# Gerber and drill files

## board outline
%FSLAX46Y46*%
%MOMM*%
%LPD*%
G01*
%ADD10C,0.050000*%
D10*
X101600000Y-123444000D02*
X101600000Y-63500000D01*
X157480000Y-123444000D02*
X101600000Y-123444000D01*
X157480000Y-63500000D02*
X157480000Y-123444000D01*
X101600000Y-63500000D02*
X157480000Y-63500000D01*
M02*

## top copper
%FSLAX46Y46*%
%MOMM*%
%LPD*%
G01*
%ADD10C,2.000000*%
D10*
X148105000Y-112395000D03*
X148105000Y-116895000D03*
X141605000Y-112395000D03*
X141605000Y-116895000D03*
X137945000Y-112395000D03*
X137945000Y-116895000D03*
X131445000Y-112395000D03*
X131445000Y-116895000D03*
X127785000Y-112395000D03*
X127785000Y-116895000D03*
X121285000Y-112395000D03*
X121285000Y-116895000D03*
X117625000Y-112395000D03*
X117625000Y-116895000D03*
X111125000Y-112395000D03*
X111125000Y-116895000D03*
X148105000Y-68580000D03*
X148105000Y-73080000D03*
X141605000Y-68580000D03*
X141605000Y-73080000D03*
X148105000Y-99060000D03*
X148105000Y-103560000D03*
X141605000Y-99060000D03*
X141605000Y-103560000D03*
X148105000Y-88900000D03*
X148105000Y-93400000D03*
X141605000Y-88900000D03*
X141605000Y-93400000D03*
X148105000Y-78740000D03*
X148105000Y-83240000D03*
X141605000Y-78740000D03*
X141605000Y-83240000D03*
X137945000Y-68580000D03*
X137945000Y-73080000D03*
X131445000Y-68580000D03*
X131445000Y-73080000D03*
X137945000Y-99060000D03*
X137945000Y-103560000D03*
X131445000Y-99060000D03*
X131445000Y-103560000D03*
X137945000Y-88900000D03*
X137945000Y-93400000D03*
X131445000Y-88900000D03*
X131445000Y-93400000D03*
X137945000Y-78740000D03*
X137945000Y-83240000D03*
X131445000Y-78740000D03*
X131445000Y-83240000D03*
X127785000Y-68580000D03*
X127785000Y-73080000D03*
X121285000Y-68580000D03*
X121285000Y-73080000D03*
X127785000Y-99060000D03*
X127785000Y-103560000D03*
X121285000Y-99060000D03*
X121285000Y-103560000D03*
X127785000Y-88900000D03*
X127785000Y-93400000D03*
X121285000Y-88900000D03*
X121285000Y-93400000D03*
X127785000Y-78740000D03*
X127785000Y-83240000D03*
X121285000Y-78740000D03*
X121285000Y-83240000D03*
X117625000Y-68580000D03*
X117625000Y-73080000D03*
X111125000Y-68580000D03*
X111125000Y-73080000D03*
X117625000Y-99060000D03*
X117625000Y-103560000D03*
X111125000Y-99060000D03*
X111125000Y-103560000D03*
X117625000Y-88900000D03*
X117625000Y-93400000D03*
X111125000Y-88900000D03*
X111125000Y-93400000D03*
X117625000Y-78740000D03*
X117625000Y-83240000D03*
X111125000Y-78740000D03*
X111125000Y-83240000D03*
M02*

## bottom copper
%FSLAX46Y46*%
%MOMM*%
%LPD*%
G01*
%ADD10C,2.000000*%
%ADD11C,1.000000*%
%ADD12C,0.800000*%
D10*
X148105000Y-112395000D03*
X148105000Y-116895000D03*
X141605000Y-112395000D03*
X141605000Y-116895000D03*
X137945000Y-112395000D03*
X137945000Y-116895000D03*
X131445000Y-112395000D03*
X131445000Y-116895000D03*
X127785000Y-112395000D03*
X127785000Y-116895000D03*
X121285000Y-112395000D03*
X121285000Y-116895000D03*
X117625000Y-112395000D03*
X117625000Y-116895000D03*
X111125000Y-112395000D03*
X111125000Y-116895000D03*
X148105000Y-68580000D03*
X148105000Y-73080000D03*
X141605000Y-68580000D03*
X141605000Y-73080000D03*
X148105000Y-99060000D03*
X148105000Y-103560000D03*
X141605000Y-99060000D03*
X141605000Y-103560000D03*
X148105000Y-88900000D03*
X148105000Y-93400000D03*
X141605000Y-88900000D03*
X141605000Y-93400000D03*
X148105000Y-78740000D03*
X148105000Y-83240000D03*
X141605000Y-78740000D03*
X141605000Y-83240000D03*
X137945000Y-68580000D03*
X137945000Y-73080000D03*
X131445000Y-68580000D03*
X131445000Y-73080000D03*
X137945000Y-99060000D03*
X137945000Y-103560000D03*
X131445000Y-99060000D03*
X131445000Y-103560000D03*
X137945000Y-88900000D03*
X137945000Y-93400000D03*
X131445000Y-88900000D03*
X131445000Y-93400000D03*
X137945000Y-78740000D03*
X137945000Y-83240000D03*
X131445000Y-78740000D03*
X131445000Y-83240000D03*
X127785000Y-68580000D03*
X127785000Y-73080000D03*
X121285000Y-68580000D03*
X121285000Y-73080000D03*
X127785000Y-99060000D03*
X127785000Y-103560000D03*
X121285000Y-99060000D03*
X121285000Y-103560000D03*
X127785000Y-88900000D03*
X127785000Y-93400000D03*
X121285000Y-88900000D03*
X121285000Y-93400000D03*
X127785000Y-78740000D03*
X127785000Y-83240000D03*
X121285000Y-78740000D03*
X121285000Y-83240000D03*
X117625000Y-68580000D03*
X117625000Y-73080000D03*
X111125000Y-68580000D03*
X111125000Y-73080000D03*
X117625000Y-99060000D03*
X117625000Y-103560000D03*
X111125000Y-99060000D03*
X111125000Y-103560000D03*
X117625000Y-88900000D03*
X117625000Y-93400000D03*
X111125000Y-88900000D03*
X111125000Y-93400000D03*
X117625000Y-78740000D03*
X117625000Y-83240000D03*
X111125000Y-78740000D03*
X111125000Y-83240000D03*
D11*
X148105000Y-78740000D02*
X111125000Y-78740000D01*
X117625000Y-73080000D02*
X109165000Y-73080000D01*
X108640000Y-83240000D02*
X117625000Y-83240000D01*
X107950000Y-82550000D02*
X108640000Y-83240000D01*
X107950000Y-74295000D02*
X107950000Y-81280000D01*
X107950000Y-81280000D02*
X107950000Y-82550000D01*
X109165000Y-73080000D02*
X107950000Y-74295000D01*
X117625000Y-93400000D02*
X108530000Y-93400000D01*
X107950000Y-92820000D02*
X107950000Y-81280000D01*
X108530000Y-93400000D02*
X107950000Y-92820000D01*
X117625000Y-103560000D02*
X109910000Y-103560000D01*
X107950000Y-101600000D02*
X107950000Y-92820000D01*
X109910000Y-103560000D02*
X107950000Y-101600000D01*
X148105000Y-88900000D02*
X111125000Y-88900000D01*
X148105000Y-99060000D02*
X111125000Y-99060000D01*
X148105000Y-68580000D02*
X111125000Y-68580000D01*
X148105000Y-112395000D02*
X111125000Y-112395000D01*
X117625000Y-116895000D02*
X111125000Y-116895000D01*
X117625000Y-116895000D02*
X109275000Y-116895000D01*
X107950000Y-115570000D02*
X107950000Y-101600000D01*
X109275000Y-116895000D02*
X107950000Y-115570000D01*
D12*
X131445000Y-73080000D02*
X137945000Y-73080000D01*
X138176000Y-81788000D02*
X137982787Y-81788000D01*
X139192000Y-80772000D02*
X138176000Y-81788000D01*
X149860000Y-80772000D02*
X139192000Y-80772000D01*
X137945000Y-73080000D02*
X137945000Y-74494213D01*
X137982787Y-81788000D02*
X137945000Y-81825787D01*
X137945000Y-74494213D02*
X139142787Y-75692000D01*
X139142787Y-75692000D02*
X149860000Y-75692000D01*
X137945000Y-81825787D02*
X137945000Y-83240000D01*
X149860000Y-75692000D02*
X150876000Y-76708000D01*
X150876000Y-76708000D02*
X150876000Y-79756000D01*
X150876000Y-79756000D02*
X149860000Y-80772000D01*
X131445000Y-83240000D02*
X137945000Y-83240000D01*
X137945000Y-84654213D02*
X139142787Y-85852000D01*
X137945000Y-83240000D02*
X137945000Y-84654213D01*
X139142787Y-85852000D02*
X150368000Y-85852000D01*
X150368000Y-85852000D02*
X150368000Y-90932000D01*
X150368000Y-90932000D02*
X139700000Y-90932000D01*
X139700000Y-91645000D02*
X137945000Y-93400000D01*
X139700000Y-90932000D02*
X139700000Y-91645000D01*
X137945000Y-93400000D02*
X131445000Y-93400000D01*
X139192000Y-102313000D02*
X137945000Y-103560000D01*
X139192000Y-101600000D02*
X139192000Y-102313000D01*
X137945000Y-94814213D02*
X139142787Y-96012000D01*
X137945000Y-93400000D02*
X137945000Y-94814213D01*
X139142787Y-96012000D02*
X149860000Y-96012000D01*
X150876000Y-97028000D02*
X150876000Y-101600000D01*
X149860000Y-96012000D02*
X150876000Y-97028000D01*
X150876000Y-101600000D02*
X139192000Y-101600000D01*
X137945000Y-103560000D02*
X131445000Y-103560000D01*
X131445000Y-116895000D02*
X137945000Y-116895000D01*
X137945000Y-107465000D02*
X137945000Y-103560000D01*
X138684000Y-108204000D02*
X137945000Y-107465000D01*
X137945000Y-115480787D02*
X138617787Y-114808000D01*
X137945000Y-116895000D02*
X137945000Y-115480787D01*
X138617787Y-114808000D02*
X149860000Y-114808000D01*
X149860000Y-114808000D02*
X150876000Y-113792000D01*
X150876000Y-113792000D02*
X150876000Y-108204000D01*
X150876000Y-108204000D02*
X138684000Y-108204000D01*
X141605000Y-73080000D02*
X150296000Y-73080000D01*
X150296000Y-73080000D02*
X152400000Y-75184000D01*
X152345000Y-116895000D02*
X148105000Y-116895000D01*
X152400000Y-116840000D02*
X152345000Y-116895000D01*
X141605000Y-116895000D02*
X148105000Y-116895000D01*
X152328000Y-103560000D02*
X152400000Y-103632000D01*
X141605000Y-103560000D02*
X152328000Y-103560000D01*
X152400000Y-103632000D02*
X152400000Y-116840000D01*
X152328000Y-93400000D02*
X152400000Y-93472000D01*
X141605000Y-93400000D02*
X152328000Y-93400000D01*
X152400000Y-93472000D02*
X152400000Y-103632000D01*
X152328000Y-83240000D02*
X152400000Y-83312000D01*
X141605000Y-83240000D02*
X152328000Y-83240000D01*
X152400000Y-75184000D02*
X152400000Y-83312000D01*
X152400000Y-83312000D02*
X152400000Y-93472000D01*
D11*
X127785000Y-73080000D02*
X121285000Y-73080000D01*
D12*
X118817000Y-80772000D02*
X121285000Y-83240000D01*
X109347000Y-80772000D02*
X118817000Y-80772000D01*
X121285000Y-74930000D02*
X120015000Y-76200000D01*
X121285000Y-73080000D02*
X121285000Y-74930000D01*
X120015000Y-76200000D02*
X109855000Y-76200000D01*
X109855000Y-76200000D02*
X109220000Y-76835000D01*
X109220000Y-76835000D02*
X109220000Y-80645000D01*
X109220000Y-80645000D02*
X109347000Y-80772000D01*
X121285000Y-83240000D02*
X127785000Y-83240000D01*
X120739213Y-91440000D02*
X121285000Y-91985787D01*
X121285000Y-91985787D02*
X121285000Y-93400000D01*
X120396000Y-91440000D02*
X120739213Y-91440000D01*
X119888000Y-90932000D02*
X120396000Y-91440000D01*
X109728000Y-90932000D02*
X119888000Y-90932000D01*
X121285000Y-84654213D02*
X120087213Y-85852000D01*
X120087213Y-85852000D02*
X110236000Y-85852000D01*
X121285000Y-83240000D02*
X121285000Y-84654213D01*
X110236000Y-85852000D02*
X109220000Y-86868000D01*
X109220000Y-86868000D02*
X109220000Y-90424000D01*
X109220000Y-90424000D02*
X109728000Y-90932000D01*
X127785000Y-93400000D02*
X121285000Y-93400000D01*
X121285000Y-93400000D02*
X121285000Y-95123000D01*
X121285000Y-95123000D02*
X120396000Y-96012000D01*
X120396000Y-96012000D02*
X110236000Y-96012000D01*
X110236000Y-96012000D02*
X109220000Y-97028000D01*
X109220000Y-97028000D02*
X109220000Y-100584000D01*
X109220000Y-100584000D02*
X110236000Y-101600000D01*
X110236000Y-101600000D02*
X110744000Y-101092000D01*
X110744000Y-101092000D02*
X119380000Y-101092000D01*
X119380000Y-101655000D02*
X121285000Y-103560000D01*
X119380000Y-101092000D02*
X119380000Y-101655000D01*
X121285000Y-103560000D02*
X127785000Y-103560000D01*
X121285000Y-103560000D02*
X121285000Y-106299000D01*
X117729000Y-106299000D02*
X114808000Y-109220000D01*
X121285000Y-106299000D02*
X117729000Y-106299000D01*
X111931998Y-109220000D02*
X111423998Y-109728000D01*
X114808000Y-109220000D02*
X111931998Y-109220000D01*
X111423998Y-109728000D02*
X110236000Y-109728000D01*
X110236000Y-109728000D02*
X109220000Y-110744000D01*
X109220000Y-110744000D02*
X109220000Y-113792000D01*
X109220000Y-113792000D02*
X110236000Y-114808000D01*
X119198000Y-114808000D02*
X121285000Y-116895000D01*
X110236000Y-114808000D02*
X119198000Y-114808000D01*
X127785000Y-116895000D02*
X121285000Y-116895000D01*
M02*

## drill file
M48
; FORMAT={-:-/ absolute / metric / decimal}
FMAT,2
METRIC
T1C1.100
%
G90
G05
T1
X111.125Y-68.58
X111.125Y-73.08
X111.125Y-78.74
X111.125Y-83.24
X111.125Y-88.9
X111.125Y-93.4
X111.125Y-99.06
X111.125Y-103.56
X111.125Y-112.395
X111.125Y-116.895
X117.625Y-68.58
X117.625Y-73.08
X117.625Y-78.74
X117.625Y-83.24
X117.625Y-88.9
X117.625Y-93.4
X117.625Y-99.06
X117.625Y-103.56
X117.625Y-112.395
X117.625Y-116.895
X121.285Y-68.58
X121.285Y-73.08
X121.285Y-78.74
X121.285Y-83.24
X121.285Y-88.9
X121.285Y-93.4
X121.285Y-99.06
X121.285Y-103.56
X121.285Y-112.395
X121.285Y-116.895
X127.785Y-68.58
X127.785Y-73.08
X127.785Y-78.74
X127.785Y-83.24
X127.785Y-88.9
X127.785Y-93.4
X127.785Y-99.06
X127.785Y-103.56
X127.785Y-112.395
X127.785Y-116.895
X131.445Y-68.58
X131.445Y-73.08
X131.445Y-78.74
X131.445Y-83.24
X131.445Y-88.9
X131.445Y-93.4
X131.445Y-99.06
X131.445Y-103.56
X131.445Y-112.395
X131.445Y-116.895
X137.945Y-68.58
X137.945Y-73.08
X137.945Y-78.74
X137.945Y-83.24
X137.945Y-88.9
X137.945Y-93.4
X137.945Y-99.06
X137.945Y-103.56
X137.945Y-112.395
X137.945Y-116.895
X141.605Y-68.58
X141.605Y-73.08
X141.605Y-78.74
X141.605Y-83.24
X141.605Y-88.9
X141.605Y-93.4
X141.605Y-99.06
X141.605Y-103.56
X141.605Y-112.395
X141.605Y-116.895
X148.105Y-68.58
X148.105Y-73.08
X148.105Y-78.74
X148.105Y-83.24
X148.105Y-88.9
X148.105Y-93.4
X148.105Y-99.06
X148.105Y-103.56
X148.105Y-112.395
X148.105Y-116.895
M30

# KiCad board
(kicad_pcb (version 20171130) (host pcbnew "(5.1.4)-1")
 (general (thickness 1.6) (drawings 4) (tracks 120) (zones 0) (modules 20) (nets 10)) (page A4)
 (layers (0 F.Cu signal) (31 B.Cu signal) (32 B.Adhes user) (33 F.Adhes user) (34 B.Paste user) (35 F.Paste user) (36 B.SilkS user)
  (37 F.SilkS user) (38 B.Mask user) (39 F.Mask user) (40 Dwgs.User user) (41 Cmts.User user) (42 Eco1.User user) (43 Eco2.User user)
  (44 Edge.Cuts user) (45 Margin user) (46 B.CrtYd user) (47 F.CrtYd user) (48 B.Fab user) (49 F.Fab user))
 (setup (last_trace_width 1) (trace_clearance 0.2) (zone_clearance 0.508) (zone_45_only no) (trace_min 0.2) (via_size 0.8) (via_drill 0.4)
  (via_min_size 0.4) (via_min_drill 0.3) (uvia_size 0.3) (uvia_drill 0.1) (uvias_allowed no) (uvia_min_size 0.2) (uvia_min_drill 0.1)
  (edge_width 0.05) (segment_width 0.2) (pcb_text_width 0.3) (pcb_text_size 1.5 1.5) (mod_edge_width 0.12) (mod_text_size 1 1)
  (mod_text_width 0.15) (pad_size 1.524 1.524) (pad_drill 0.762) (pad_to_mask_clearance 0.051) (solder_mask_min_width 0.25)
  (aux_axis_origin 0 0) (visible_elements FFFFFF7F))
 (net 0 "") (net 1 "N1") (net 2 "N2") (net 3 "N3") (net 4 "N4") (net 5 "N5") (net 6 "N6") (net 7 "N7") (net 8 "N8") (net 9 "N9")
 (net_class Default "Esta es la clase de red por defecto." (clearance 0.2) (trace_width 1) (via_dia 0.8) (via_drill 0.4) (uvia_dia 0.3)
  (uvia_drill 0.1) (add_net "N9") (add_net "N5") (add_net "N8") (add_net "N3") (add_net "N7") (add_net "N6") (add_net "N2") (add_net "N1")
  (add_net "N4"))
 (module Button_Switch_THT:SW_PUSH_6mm (layer F.Cu) (at 141.605 112.395)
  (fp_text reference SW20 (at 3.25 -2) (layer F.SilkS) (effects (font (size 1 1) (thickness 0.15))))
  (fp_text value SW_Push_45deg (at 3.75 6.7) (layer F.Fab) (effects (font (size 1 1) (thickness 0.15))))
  (pad 1 thru_hole circle (at 6.5 0 90) (size 2 2) (drill 1.1) (layers *.Cu *.Mask) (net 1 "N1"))
  (pad 2 thru_hole circle (at 6.5 4.5 90) (size 2 2) (drill 1.1) (layers *.Cu *.Mask) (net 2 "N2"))
  (pad 1 thru_hole circle (at 0 0 90) (size 2 2) (drill 1.1) (layers *.Cu *.Mask) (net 1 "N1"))
  (pad 2 thru_hole circle (at 0 4.5 90) (size 2 2) (drill 1.1) (layers *.Cu *.Mask) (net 2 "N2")))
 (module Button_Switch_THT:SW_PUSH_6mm (layer F.Cu) (at 131.445 112.395)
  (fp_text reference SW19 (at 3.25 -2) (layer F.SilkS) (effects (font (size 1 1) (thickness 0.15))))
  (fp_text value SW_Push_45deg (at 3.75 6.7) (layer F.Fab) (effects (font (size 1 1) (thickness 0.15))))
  (pad 1 thru_hole circle (at 6.5 0 90) (size 2 2) (drill 1.1) (layers *.Cu *.Mask) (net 1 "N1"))
  (pad 2 thru_hole circle (at 6.5 4.5 90) (size 2 2) (drill 1.1) (layers *.Cu *.Mask) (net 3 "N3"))
  (pad 1 thru_hole circle (at 0 0 90) (size 2 2) (drill 1.1) (layers *.Cu *.Mask) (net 1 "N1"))
  (pad 2 thru_hole circle (at 0 4.5 90) (size 2 2) (drill 1.1) (layers *.Cu *.Mask) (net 3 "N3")))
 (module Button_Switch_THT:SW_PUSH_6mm (layer F.Cu) (at 121.285 112.395)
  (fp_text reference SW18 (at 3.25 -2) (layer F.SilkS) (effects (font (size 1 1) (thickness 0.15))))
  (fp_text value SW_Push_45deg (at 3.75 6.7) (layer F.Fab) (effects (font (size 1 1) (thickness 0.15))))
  (pad 1 thru_hole circle (at 6.5 0 90) (size 2 2) (drill 1.1) (layers *.Cu *.Mask) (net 1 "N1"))
  (pad 2 thru_hole circle (at 6.5 4.5 90) (size 2 2) (drill 1.1) (layers *.Cu *.Mask) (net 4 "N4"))
  (pad 1 thru_hole circle (at 0 0 90) (size 2 2) (drill 1.1) (layers *.Cu *.Mask) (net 1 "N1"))
  (pad 2 thru_hole circle (at 0 4.5 90) (size 2 2) (drill 1.1) (layers *.Cu *.Mask) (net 4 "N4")))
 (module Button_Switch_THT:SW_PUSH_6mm (layer F.Cu) (at 111.125 112.395)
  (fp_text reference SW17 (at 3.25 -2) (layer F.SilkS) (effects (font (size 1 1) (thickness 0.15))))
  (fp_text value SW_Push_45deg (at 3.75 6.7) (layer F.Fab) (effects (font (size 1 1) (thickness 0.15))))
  (pad 1 thru_hole circle (at 6.5 0 90) (size 2 2) (drill 1.1) (layers *.Cu *.Mask) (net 1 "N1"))
  (pad 2 thru_hole circle (at 6.5 4.5 90) (size 2 2) (drill 1.1) (layers *.Cu *.Mask) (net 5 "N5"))
  (pad 1 thru_hole circle (at 0 0 90) (size 2 2) (drill 1.1) (layers *.Cu *.Mask) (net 1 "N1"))
  (pad 2 thru_hole circle (at 0 4.5 90) (size 2 2) (drill 1.1) (layers *.Cu *.Mask) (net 5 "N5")))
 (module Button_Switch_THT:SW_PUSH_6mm (layer F.Cu) (at 141.605 68.58)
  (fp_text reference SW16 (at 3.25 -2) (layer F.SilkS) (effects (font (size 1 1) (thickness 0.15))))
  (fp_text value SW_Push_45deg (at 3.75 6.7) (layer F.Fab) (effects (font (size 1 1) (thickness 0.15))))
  (pad 1 thru_hole circle (at 6.5 0 90) (size 2 2) (drill 1.1) (layers *.Cu *.Mask) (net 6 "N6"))
  (pad 2 thru_hole circle (at 6.5 4.5 90) (size 2 2) (drill 1.1) (layers *.Cu *.Mask) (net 2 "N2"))
  (pad 1 thru_hole circle (at 0 0 90) (size 2 2) (drill 1.1) (layers *.Cu *.Mask) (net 6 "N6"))
  (pad 2 thru_hole circle (at 0 4.5 90) (size 2 2) (drill 1.1) (layers *.Cu *.Mask) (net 2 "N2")))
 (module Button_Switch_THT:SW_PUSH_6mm (layer F.Cu) (at 141.605 99.06)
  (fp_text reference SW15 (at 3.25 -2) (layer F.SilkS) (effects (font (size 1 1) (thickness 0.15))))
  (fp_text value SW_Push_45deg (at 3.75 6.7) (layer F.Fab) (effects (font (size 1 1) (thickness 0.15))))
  (pad 1 thru_hole circle (at 6.5 0 90) (size 2 2) (drill 1.1) (layers *.Cu *.Mask) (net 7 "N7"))
  (pad 2 thru_hole circle (at 6.5 4.5 90) (size 2 2) (drill 1.1) (layers *.Cu *.Mask) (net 2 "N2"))
  (pad 1 thru_hole circle (at 0 0 90) (size 2 2) (drill 1.1) (layers *.Cu *.Mask) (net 7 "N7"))
  (pad 2 thru_hole circle (at 0 4.5 90) (size 2 2) (drill 1.1) (layers *.Cu *.Mask) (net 2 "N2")))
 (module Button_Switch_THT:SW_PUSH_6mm (layer F.Cu) (at 141.605 88.9)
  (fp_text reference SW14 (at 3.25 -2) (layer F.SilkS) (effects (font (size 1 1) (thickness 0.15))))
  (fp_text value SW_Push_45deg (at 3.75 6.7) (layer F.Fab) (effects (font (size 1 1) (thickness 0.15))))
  (pad 1 thru_hole circle (at 6.5 0 90) (size 2 2) (drill 1.1) (layers *.Cu *.Mask) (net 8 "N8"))
  (pad 2 thru_hole circle (at 6.5 4.5 90) (size 2 2) (drill 1.1) (layers *.Cu *.Mask) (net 2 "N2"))
  (pad 1 thru_hole circle (at 0 0 90) (size 2 2) (drill 1.1) (layers *.Cu *.Mask) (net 8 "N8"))
  (pad 2 thru_hole circle (at 0 4.5 90) (size 2 2) (drill 1.1) (layers *.Cu *.Mask) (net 2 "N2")))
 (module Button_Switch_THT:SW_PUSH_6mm (layer F.Cu) (at 141.605 78.74)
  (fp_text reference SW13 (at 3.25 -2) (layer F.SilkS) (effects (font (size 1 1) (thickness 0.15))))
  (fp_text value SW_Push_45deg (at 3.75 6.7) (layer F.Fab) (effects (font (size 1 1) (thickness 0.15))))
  (pad 1 thru_hole circle (at 6.5 0 90) (size 2 2) (drill 1.1) (layers *.Cu *.Mask) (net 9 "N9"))
  (pad 2 thru_hole circle (at 6.5 4.5 90) (size 2 2) (drill 1.1) (layers *.Cu *.Mask) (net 2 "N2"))
  (pad 1 thru_hole circle (at 0 0 90) (size 2 2) (drill 1.1) (layers *.Cu *.Mask) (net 9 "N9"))
  (pad 2 thru_hole circle (at 0 4.5 90) (size 2 2) (drill 1.1) (layers *.Cu *.Mask) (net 2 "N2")))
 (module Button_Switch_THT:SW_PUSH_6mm (layer F.Cu) (at 131.445 68.58)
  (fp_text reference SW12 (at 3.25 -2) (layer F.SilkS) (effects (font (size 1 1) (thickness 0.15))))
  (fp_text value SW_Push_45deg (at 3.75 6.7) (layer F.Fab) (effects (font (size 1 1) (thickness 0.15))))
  (pad 1 thru_hole circle (at 6.5 0 90) (size 2 2) (drill 1.1) (layers *.Cu *.Mask) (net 6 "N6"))
  (pad 2 thru_hole circle (at 6.5 4.5 90) (size 2 2) (drill 1.1) (layers *.Cu *.Mask) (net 3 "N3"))
  (pad 1 thru_hole circle (at 0 0 90) (size 2 2) (drill 1.1) (layers *.Cu *.Mask) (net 6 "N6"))
  (pad 2 thru_hole circle (at 0 4.5 90) (size 2 2) (drill 1.1) (layers *.Cu *.Mask) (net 3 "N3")))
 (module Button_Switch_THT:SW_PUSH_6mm (layer F.Cu) (at 131.445 99.06)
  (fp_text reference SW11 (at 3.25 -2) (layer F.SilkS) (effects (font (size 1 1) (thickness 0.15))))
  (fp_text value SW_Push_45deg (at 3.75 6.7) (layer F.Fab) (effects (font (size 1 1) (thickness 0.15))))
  (pad 1 thru_hole circle (at 6.5 0 90) (size 2 2) (drill 1.1) (layers *.Cu *.Mask) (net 7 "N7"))
  (pad 2 thru_hole circle (at 6.5 4.5 90) (size 2 2) (drill 1.1) (layers *.Cu *.Mask) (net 3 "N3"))
  (pad 1 thru_hole circle (at 0 0 90) (size 2 2) (drill 1.1) (layers *.Cu *.Mask) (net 7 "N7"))
  (pad 2 thru_hole circle (at 0 4.5 90) (size 2 2) (drill 1.1) (layers *.Cu *.Mask) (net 3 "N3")))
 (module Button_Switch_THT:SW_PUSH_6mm (layer F.Cu) (at 131.445 88.9)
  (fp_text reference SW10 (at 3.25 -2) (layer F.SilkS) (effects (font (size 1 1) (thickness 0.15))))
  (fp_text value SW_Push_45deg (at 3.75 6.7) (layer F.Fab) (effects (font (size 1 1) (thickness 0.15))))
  (pad 1 thru_hole circle (at 6.5 0 90) (size 2 2) (drill 1.1) (layers *.Cu *.Mask) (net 8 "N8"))
  (pad 2 thru_hole circle (at 6.5 4.5 90) (size 2 2) (drill 1.1) (layers *.Cu *.Mask) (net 3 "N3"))
  (pad 1 thru_hole circle (at 0 0 90) (size 2 2) (drill 1.1) (layers *.Cu *.Mask) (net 8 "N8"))
  (pad 2 thru_hole circle (at 0 4.5 90) (size 2 2) (drill 1.1) (layers *.Cu *.Mask) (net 3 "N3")))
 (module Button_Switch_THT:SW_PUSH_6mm (layer F.Cu) (at 131.445 78.74)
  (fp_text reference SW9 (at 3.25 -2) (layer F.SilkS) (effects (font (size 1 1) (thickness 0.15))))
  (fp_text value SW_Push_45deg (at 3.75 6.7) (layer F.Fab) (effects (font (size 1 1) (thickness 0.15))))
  (pad 1 thru_hole circle (at 6.5 0 90) (size 2 2) (drill 1.1) (layers *.Cu *.Mask) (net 9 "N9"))
  (pad 2 thru_hole circle (at 6.5 4.5 90) (size 2 2) (drill 1.1) (layers *.Cu *.Mask) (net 3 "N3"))
  (pad 1 thru_hole circle (at 0 0 90) (size 2 2) (drill 1.1) (layers *.Cu *.Mask) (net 9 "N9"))
  (pad 2 thru_hole circle (at 0 4.5 90) (size 2 2) (drill 1.1) (layers *.Cu *.Mask) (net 3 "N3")))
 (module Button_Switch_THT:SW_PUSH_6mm (layer F.Cu) (at 121.285 68.58)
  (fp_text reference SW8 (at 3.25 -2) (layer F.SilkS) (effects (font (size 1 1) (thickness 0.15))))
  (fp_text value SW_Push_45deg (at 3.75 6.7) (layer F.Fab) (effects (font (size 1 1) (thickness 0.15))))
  (pad 1 thru_hole circle (at 6.5 0 90) (size 2 2) (drill 1.1) (layers *.Cu *.Mask) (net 6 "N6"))
  (pad 2 thru_hole circle (at 6.5 4.5 90) (size 2 2) (drill 1.1) (layers *.Cu *.Mask) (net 4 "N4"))
  (pad 1 thru_hole circle (at 0 0 90) (size 2 2) (drill 1.1) (layers *.Cu *.Mask) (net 6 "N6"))
  (pad 2 thru_hole circle (at 0 4.5 90) (size 2 2) (drill 1.1) (layers *.Cu *.Mask) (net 4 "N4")))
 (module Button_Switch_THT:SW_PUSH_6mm (layer F.Cu) (at 121.285 99.06)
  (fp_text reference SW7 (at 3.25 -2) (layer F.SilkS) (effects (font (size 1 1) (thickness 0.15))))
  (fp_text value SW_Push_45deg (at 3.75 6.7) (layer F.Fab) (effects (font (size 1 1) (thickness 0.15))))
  (pad 1 thru_hole circle (at 6.5 0 90) (size 2 2) (drill 1.1) (layers *.Cu *.Mask) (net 7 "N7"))
  (pad 2 thru_hole circle (at 6.5 4.5 90) (size 2 2) (drill 1.1) (layers *.Cu *.Mask) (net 4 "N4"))
  (pad 1 thru_hole circle (at 0 0 90) (size 2 2) (drill 1.1) (layers *.Cu *.Mask) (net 7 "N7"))
  (pad 2 thru_hole circle (at 0 4.5 90) (size 2 2) (drill 1.1) (layers *.Cu *.Mask) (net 4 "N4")))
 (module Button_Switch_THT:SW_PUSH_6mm (layer F.Cu) (at 121.285 88.9)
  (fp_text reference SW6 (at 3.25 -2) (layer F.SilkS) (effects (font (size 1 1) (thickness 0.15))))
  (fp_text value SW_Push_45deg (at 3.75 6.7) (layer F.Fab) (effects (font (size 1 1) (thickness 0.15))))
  (pad 1 thru_hole circle (at 6.5 0 90) (size 2 2) (drill 1.1) (layers *.Cu *.Mask) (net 8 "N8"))
  (pad 2 thru_hole circle (at 6.5 4.5 90) (size 2 2) (drill 1.1) (layers *.Cu *.Mask) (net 4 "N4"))
  (pad 1 thru_hole circle (at 0 0 90) (size 2 2) (drill 1.1) (layers *.Cu *.Mask) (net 8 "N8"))
  (pad 2 thru_hole circle (at 0 4.5 90) (size 2 2) (drill 1.1) (layers *.Cu *.Mask) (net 4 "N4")))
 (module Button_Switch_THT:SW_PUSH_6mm (layer F.Cu) (at 121.285 78.74)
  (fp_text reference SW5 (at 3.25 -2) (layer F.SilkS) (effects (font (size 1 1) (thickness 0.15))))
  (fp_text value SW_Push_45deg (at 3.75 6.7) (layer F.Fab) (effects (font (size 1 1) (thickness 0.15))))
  (pad 1 thru_hole circle (at 6.5 0 90) (size 2 2) (drill 1.1) (layers *.Cu *.Mask) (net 9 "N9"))
  (pad 2 thru_hole circle (at 6.5 4.5 90) (size 2 2) (drill 1.1) (layers *.Cu *.Mask) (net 4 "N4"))
  (pad 1 thru_hole circle (at 0 0 90) (size 2 2) (drill 1.1) (layers *.Cu *.Mask) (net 9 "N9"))
  (pad 2 thru_hole circle (at 0 4.5 90) (size 2 2) (drill 1.1) (layers *.Cu *.Mask) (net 4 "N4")))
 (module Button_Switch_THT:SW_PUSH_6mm (layer F.Cu) (at 111.125 68.58)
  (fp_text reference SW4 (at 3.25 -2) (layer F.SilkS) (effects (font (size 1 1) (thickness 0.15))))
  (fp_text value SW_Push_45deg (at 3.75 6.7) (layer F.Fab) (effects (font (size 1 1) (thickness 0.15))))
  (pad 1 thru_hole circle (at 6.5 0 90) (size 2 2) (drill 1.1) (layers *.Cu *.Mask) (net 6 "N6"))
  (pad 2 thru_hole circle (at 6.5 4.5 90) (size 2 2) (drill 1.1) (layers *.Cu *.Mask) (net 5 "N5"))
  (pad 1 thru_hole circle (at 0 0 90) (size 2 2) (drill 1.1) (layers *.Cu *.Mask) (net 6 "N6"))
  (pad 2 thru_hole circle (at 0 4.5 90) (size 2 2) (drill 1.1) (layers *.Cu *.Mask) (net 5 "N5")))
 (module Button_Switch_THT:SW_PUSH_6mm (layer F.Cu) (at 111.125 99.06)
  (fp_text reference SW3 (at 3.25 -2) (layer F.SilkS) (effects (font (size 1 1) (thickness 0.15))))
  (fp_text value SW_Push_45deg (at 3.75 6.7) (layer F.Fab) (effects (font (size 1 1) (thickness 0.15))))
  (pad 1 thru_hole circle (at 6.5 0 90) (size 2 2) (drill 1.1) (layers *.Cu *.Mask) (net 7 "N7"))
  (pad 2 thru_hole circle (at 6.5 4.5 90) (size 2 2) (drill 1.1) (layers *.Cu *.Mask) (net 5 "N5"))
  (pad 1 thru_hole circle (at 0 0 90) (size 2 2) (drill 1.1) (layers *.Cu *.Mask) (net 7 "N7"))
  (pad 2 thru_hole circle (at 0 4.5 90) (size 2 2) (drill 1.1) (layers *.Cu *.Mask) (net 5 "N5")))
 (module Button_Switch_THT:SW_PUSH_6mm (layer F.Cu) (at 111.125 88.9)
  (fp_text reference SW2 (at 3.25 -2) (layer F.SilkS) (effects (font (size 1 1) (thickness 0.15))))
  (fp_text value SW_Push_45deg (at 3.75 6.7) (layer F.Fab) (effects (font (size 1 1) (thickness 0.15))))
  (pad 1 thru_hole circle (at 6.5 0 90) (size 2 2) (drill 1.1) (layers *.Cu *.Mask) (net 8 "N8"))
  (pad 2 thru_hole circle (at 6.5 4.5 90) (size 2 2) (drill 1.1) (layers *.Cu *.Mask) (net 5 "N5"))
  (pad 1 thru_hole circle (at 0 0 90) (size 2 2) (drill 1.1) (layers *.Cu *.Mask) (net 8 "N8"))
  (pad 2 thru_hole circle (at 0 4.5 90) (size 2 2) (drill 1.1) (layers *.Cu *.Mask) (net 5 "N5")))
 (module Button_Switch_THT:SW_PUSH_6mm (layer F.Cu) (at 111.125 78.74)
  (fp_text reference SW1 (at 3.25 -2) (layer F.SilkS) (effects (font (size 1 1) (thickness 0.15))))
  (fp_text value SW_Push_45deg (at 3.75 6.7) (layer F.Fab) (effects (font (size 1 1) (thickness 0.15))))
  (pad 1 thru_hole circle (at 6.5 0 90) (size 2 2) (drill 1.1) (layers *.Cu *.Mask) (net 9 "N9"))
  (pad 2 thru_hole circle (at 6.5 4.5 90) (size 2 2) (drill 1.1) (layers *.Cu *.Mask) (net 5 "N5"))
  (pad 1 thru_hole circle (at 0 0 90) (size 2 2) (drill 1.1) (layers *.Cu *.Mask) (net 9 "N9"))
  (pad 2 thru_hole circle (at 0 4.5 90) (size 2 2) (drill 1.1) (layers *.Cu *.Mask) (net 5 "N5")))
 (gr_line (start 101.6 123.444) (end 101.6 63.5) (layer Edge.Cuts) (width 0.05))
 (gr_line (start 157.48 123.444) (end 101.6 123.444) (layer Edge.Cuts) (width 0.05))
 (gr_line (start 157.48 63.5) (end 157.48 123.444) (layer Edge.Cuts) (width 0.05))
 (gr_line (start 101.6 63.5) (end 157.48 63.5) (layer Edge.Cuts) (width 0.05))
 (segment (start 148.105 78.74) (end 111.125 78.74) (width 1) (layer B.Cu) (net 9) (status C00000))
 (segment (start 117.625 73.08) (end 109.165 73.08) (width 1) (layer B.Cu) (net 5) (status 400000))
 (segment (start 108.64 83.24) (end 117.625 83.24) (width 1) (layer B.Cu) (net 5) (status 800000))
 (segment (start 107.95 82.55) (end 108.64 83.24) (width 1) (layer B.Cu) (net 5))
 (segment (start 107.95 74.295) (end 107.95 81.28) (width 1) (layer B.Cu) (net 5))
 (segment (start 107.95 81.28) (end 107.95 82.55) (width 1) (layer B.Cu) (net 5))
 (segment (start 109.165 73.08) (end 107.95 74.295) (width 1) (layer B.Cu) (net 5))
 (segment (start 117.625 93.4) (end 108.53 93.4) (width 1) (layer B.Cu) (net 5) (status 400000))
 (segment (start 107.95 92.82) (end 107.95 81.28) (width 1) (layer B.Cu) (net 5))
 (segment (start 108.53 93.4) (end 107.95 92.82) (width 1) (layer B.Cu) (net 5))
 (segment (start 117.625 103.56) (end 109.91 103.56) (width 1) (layer B.Cu) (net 5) (status 400000))
 (segment (start 107.95 101.6) (end 107.95 92.82) (width 1) (layer B.Cu) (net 5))
 (segment (start 109.91 103.56) (end 107.95 101.6) (width 1) (layer B.Cu) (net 5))
 (segment (start 148.105 88.9) (end 111.125 88.9) (width 1) (layer B.Cu) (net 8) (status C00000))
 (segment (start 148.105 99.06) (end 111.125 99.06) (width 1) (layer B.Cu) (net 7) (status C00000))
 (segment (start 148.105 68.58) (end 111.125 68.58) (width 1) (layer B.Cu) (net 6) (status C00000))
 (segment (start 148.105 112.395) (end 111.125 112.395) (width 1) (layer B.Cu) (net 1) (status C00000))
 (segment (start 117.625 116.895) (end 111.125 116.895) (width 1) (layer B.Cu) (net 5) (status C00000))
 (segment (start 117.625 116.895) (end 109.275 116.895) (width 1) (layer B.Cu) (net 5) (status 400000))
 (segment (start 107.95 115.57) (end 107.95 101.6) (width 1) (layer B.Cu) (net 5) (status 1000000))
 (segment (start 109.275 116.895) (end 107.95 115.57) (width 1) (layer B.Cu) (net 5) (status 1000000))
 (segment (start 131.445 73.08) (end 137.945 73.08) (width 0.8) (layer B.Cu) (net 3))
 (segment (start 138.176 81.788) (end 137.982787 81.788) (width 0.8) (layer B.Cu) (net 3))
 (segment (start 139.192 80.772) (end 138.176 81.788) (width 0.8) (layer B.Cu) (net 3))
 (segment (start 149.86 80.772) (end 139.192 80.772) (width 0.8) (layer B.Cu) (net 3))
 (segment (start 137.945 73.08) (end 137.945 74.494213) (width 0.8) (layer B.Cu) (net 3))
 (segment (start 137.982787 81.788) (end 137.945 81.825787) (width 0.8) (layer B.Cu) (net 3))
 (segment (start 137.945 74.494213) (end 139.142787 75.692) (width 0.8) (layer B.Cu) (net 3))
 (segment (start 139.142787 75.692) (end 149.86 75.692) (width 0.8) (layer B.Cu) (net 3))
 (segment (start 137.945 81.825787) (end 137.945 83.24) (width 0.8) (layer B.Cu) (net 3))
 (segment (start 149.86 75.692) (end 150.876 76.708) (width 0.8) (layer B.Cu) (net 3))
 (segment (start 150.876 76.708) (end 150.876 79.756) (width 0.8) (layer B.Cu) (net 3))
 (segment (start 150.876 79.756) (end 149.86 80.772) (width 0.8) (layer B.Cu) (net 3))
 (segment (start 131.445 83.24) (end 137.945 83.24) (width 0.8) (layer B.Cu) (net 3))
 (segment (start 137.945 84.654213) (end 139.142787 85.852) (width 0.8) (layer B.Cu) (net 3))
 (segment (start 137.945 83.24) (end 137.945 84.654213) (width 0.8) (layer B.Cu) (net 3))
 (segment (start 139.142787 85.852) (end 150.368 85.852) (width 0.8) (layer B.Cu) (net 3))
 (segment (start 150.368 85.852) (end 150.368 90.932) (width 0.8) (layer B.Cu) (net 3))
 (segment (start 150.368 90.932) (end 139.7 90.932) (width 0.8) (layer B.Cu) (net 3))
 (segment (start 139.7 91.645) (end 137.945 93.4) (width 0.8) (layer B.Cu) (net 3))
 (segment (start 139.7 90.932) (end 139.7 91.645) (width 0.8) (layer B.Cu) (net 3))
 (segment (start 137.945 93.4) (end 131.445 93.4) (width 0.8) (layer B.Cu) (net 3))
 (segment (start 139.192 102.313) (end 137.945 103.56) (width 0.8) (layer B.Cu) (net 3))
 (segment (start 139.192 101.6) (end 139.192 102.313) (width 0.8) (layer B.Cu) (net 3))
 (segment (start 137.945 94.814213) (end 139.142787 96.012) (width 0.8) (layer B.Cu) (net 3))
 (segment (start 137.945 93.4) (end 137.945 94.814213) (width 0.8) (layer B.Cu) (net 3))
 (segment (start 139.142787 96.012) (end 149.86 96.012) (width 0.8) (layer B.Cu) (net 3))
 (segment (start 150.876 97.028) (end 150.876 101.6) (width 0.8) (layer B.Cu) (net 3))
 (segment (start 149.86 96.012) (end 150.876 97.028) (width 0.8) (layer B.Cu) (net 3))
 (segment (start 150.876 101.6) (end 139.192 101.6) (width 0.8) (layer B.Cu) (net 3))
 (segment (start 137.945 103.56) (end 131.445 103.56) (width 0.8) (layer B.Cu) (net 3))
 (segment (start 131.445 116.895) (end 137.945 116.895) (width 0.8) (layer B.Cu) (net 3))
 (segment (start 137.945 107.465) (end 137.945 103.56) (width 0.8) (layer B.Cu) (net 3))
 (segment (start 138.684 108.204) (end 137.945 107.465) (width 0.8) (layer B.Cu) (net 3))
 (segment (start 137.945 115.480787) (end 138.617787 114.808) (width 0.8) (layer B.Cu) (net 3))
 (segment (start 137.945 116.895) (end 137.945 115.480787) (width 0.8) (layer B.Cu) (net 3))
 (segment (start 138.617787 114.808) (end 149.86 114.808) (width 0.8) (layer B.Cu) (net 3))
 (segment (start 149.86 114.808) (end 150.876 113.792) (width 0.8) (layer B.Cu) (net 3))
 (segment (start 150.876 113.792) (end 150.876 108.204) (width 0.8) (layer B.Cu) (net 3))
 (segment (start 150.876 108.204) (end 138.684 108.204) (width 0.8) (layer B.Cu) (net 3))
 (segment (start 141.605 73.08) (end 150.296 73.08) (width 0.8) (layer B.Cu) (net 2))
 (segment (start 150.296 73.08) (end 152.4 75.184) (width 0.8) (layer B.Cu) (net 2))
 (segment (start 152.345 116.895) (end 148.105 116.895) (width 0.8) (layer B.Cu) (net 2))
 (segment (start 152.4 116.84) (end 152.345 116.895) (width 0.8) (layer B.Cu) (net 2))
 (segment (start 141.605 116.895) (end 148.105 116.895) (width 0.8) (layer B.Cu) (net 2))
 (segment (start 152.328 103.56) (end 152.4 103.632) (width 0.8) (layer B.Cu) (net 2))
 (segment (start 141.605 103.56) (end 152.328 103.56) (width 0.8) (layer B.Cu) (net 2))
 (segment (start 152.4 103.632) (end 152.4 116.84) (width 0.8) (layer B.Cu) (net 2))
 (segment (start 152.328 93.4) (end 152.4 93.472) (width 0.8) (layer B.Cu) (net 2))
 (segment (start 141.605 93.4) (end 152.328 93.4) (width 0.8) (layer B.Cu) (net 2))
 (segment (start 152.4 93.472) (end 152.4 103.632) (width 0.8) (layer B.Cu) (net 2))
 (segment (start 152.328 83.24) (end 152.4 83.312) (width 0.8) (layer B.Cu) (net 2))
 (segment (start 141.605 83.24) (end 152.328 83.24) (width 0.8) (layer B.Cu) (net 2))
 (segment (start 152.4 75.184) (end 152.4 83.312) (width 0.8) (layer B.Cu) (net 2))
 (segment (start 152.4 83.312) (end 152.4 93.472) (width 0.8) (layer B.Cu) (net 2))
 (segment (start 127.785 73.08) (end 121.285 73.08) (width 1) (layer B.Cu) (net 4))
 (segment (start 118.817 80.772) (end 121.285 83.24) (width 0.8) (layer B.Cu) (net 4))
 (segment (start 109.347 80.772) (end 118.817 80.772) (width 0.8) (layer B.Cu) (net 4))
 (segment (start 121.285 74.93) (end 120.015 76.2) (width 0.8) (layer B.Cu) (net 4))
 (segment (start 121.285 73.08) (end 121.285 74.93) (width 0.8) (layer B.Cu) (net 4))
 (segment (start 120.015 76.2) (end 109.855 76.2) (width 0.8) (layer B.Cu) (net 4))
 (segment (start 109.855 76.2) (end 109.22 76.835) (width 0.8) (layer B.Cu) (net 4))
 (segment (start 109.22 76.835) (end 109.22 80.645) (width 0.8) (layer B.Cu) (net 4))
 (segment (start 109.22 80.645) (end 109.347 80.772) (width 0.8) (layer B.Cu) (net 4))
 (segment (start 121.285 83.24) (end 127.785 83.24) (width 0.8) (layer B.Cu) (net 4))
 (segment (start 120.739213 91.44) (end 121.285 91.985787) (width 0.8) (layer B.Cu) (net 4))
 (segment (start 121.285 91.985787) (end 121.285 93.4) (width 0.8) (layer B.Cu) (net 4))
 (segment (start 120.396 91.44) (end 120.739213 91.44) (width 0.8) (layer B.Cu) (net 4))
 (segment (start 119.888 90.932) (end 120.396 91.44) (width 0.8) (layer B.Cu) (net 4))
 (segment (start 109.728 90.932) (end 119.888 90.932) (width 0.8) (layer B.Cu) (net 4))
 (segment (start 121.285 84.654213) (end 120.087213 85.852) (width 0.8) (layer B.Cu) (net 4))
 (segment (start 120.087213 85.852) (end 110.236 85.852) (width 0.8) (layer B.Cu) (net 4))
 (segment (start 121.285 83.24) (end 121.285 84.654213) (width 0.8) (layer B.Cu) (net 4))
 (segment (start 110.236 85.852) (end 109.22 86.868) (width 0.8) (layer B.Cu) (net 4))
 (segment (start 109.22 86.868) (end 109.22 90.424) (width 0.8) (layer B.Cu) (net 4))
 (segment (start 109.22 90.424) (end 109.728 90.932) (width 0.8) (layer B.Cu) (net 4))
 (segment (start 127.785 93.4) (end 121.285 93.4) (width 0.8) (layer B.Cu) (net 4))
 (segment (start 121.285 93.4) (end 121.285 95.123) (width 0.8) (layer B.Cu) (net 4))
 (segment (start 121.285 95.123) (end 120.396 96.012) (width 0.8) (layer B.Cu) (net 4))
 (segment (start 120.396 96.012) (end 110.236 96.012) (width 0.8) (layer B.Cu) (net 4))
 (segment (start 110.236 96.012) (end 109.22 97.028) (width 0.8) (layer B.Cu) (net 4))
 (segment (start 109.22 97.028) (end 109.22 100.584) (width 0.8) (layer B.Cu) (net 4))
 (segment (start 109.22 100.584) (end 110.236 101.6) (width 0.8) (layer B.Cu) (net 4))
 (segment (start 110.236 101.6) (end 110.744 101.092) (width 0.8) (layer B.Cu) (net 4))
 (segment (start 110.744 101.092) (end 119.38 101.092) (width 0.8) (layer B.Cu) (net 4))
 (segment (start 119.38 101.655) (end 121.285 103.56) (width 0.8) (layer B.Cu) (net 4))
 (segment (start 119.38 101.092) (end 119.38 101.655) (width 0.8) (layer B.Cu) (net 4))
 (segment (start 121.285 103.56) (end 127.785 103.56) (width 0.8) (layer B.Cu) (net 4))
 (segment (start 121.285 103.56) (end 121.285 106.299) (width 0.8) (layer B.Cu) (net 4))
 (segment (start 117.729 106.299) (end 114.808 109.22) (width 0.8) (layer B.Cu) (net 4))
 (segment (start 121.285 106.299) (end 117.729 106.299) (width 0.8) (layer B.Cu) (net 4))
 (segment (start 111.931998 109.22) (end 111.423998 109.728) (width 0.8) (layer B.Cu) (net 4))
 (segment (start 114.808 109.22) (end 111.931998 109.22) (width 0.8) (layer B.Cu) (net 4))
 (segment (start 111.423998 109.728) (end 110.236 109.728) (width 0.8) (layer B.Cu) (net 4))
 (segment (start 110.236 109.728) (end 109.22 110.744) (width 0.8) (layer B.Cu) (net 4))
 (segment (start 109.22 110.744) (end 109.22 113.792) (width 0.8) (layer B.Cu) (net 4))
 (segment (start 109.22 113.792) (end 110.236 114.808) (width 0.8) (layer B.Cu) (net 4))
 (segment (start 119.198 114.808) (end 121.285 116.895) (width 0.8) (layer B.Cu) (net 4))
 (segment (start 110.236 114.808) (end 119.198 114.808) (width 0.8) (layer B.Cu) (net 4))
 (segment (start 127.785 116.895) (end 121.285 116.895) (width 0.8) (layer B.Cu) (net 4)))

